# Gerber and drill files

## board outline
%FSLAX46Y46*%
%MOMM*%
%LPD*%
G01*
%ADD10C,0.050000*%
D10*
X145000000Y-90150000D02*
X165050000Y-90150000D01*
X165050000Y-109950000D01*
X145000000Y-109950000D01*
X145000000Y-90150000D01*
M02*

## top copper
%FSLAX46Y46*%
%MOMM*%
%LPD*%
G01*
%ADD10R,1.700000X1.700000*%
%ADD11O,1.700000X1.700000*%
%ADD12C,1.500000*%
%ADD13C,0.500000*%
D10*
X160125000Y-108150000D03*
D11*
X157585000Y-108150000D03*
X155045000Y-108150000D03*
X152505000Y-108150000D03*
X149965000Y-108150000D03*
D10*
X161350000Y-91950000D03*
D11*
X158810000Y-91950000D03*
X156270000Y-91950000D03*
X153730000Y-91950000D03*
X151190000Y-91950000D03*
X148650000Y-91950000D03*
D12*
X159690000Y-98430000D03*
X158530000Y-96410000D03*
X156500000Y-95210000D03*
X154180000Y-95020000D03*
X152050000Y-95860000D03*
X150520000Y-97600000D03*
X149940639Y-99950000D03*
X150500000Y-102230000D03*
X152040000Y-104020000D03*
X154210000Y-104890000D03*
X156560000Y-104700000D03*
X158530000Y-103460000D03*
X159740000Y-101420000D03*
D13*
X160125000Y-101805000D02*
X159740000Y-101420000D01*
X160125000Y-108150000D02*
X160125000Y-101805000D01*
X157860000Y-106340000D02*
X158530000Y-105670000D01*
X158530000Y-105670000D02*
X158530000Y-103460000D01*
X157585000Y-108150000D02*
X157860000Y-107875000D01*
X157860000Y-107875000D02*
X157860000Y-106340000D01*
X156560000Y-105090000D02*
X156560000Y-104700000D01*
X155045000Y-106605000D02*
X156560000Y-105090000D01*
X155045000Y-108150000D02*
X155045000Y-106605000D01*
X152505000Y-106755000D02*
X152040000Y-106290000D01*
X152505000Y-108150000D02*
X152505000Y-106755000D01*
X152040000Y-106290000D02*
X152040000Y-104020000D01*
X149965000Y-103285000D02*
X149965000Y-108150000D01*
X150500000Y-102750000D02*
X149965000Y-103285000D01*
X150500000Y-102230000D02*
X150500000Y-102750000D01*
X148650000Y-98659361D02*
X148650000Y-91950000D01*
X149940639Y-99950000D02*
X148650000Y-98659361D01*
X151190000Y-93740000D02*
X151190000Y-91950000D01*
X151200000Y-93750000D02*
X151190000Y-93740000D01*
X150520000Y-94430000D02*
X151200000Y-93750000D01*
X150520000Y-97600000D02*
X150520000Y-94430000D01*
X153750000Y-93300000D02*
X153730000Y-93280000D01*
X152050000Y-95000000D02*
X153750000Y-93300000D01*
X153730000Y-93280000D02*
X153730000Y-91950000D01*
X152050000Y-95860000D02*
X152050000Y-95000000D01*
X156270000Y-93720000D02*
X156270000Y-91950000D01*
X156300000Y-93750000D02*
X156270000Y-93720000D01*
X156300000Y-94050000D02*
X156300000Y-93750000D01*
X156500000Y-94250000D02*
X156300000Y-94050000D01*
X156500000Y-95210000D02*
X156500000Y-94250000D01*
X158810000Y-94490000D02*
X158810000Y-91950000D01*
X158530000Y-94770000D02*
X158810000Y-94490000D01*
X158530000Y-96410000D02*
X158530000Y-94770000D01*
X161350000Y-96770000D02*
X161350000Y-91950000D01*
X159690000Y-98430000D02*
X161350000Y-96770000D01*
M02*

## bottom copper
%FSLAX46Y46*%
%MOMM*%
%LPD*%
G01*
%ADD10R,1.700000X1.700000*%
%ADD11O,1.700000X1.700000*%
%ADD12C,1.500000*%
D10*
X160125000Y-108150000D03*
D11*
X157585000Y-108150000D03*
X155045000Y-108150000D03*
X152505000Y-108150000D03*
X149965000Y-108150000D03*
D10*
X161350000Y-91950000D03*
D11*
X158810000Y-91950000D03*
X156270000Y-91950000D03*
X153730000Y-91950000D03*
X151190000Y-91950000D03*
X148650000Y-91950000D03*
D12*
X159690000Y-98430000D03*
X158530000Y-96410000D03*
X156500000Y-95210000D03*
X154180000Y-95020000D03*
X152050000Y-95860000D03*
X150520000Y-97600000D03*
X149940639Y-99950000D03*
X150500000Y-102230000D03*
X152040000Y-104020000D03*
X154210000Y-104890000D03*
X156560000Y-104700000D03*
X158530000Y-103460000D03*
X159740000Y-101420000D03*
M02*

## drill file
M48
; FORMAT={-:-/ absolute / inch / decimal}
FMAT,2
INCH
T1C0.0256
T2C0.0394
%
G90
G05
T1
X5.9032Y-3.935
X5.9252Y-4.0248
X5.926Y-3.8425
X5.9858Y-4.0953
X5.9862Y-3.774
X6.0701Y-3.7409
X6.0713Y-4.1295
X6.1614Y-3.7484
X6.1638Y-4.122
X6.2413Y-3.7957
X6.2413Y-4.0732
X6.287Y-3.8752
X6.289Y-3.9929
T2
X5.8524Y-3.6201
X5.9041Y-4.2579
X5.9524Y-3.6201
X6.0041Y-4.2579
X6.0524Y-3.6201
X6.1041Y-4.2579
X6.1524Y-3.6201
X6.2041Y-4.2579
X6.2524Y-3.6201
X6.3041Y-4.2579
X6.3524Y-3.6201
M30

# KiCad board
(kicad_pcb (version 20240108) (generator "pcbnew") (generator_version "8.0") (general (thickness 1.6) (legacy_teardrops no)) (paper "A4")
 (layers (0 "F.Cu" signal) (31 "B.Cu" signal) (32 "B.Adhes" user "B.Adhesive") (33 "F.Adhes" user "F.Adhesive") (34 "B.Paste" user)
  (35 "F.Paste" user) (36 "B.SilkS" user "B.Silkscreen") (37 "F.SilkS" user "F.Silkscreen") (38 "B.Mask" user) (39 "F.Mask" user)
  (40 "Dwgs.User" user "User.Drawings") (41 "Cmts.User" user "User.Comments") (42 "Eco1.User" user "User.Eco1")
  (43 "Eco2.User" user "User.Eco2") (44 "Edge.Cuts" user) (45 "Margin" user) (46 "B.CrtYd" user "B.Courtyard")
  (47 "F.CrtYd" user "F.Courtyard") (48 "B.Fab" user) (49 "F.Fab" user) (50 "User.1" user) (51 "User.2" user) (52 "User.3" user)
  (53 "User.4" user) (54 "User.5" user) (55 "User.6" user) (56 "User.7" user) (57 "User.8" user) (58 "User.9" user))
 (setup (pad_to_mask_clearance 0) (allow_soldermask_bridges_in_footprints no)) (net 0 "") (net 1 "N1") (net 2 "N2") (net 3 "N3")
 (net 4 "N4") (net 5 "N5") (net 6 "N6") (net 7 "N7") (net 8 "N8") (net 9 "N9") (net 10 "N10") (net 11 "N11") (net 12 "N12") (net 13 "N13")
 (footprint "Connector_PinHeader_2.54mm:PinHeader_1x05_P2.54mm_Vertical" (layer "F.Cu") (at 160.125 108.15 -90)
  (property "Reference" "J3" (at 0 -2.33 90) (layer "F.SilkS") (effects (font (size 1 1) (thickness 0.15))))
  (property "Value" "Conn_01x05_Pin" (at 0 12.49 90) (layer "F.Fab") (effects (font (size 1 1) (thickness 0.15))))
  (pad "1" thru_hole rect (at 0 0 270) (size 1.7 1.7) (drill 1) (layers "*.Cu" "*.Mask") (remove_unused_layers no) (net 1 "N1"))
  (pad "2" thru_hole oval (at 0 2.54 270) (size 1.7 1.7) (drill 1) (layers "*.Cu" "*.Mask") (remove_unused_layers no) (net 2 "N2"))
  (pad "3" thru_hole oval (at 0 5.08 270) (size 1.7 1.7) (drill 1) (layers "*.Cu" "*.Mask") (remove_unused_layers no) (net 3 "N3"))
  (pad "4" thru_hole oval (at 0 7.62 270) (size 1.7 1.7) (drill 1) (layers "*.Cu" "*.Mask") (remove_unused_layers no) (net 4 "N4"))
  (pad "5" thru_hole oval (at 0 10.16 270) (size 1.7 1.7) (drill 1) (layers "*.Cu" "*.Mask") (remove_unused_layers no) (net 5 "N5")))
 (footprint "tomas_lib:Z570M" (layer "F.Cu") (at 154.95 99.95)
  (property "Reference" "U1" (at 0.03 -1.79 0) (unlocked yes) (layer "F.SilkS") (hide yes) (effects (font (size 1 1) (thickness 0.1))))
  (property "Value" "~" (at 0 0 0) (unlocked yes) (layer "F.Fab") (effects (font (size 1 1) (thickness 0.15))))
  (pad "1" thru_hole circle (at 4.74 -1.52) (size 1.5 1.5) (drill 0.65) (layers "*.Cu" "*.Mask") (remove_unused_layers no) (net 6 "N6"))
  (pad "2" thru_hole circle (at 3.58 -3.54) (size 1.5 1.5) (drill 0.65) (layers "*.Cu" "*.Mask") (remove_unused_layers no) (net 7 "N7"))
  (pad "3" thru_hole circle (at 1.55 -4.74) (size 1.5 1.5) (drill 0.65) (layers "*.Cu" "*.Mask") (remove_unused_layers no) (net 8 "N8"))
  (pad "4" thru_hole circle (at -0.77 -4.93) (size 1.5 1.5) (drill 0.65) (layers "*.Cu" "*.Mask") (remove_unused_layers no) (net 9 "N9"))
  (pad "5" thru_hole circle (at -2.9 -4.09) (size 1.5 1.5) (drill 0.65) (layers "*.Cu" "*.Mask") (remove_unused_layers no) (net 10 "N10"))
  (pad "6" thru_hole circle (at -4.43 -2.35) (size 1.5 1.5) (drill 0.65) (layers "*.Cu" "*.Mask") (remove_unused_layers no) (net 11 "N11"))
  (pad "7" thru_hole circle (at -5.009361 0) (size 1.5 1.5) (drill 0.65) (layers "*.Cu" "*.Mask") (remove_unused_layers no) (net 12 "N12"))
  (pad "8" thru_hole circle (at -4.45 2.28) (size 1.5 1.5) (drill 0.65) (layers "*.Cu" "*.Mask") (remove_unused_layers no) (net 5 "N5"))
  (pad "9" thru_hole circle (at -2.91 4.07) (size 1.5 1.5) (drill 0.65) (layers "*.Cu" "*.Mask") (remove_unused_layers no) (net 4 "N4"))
  (pad "10" thru_hole circle (at -0.74 4.94) (size 1.5 1.5) (drill 0.65) (layers "*.Cu" "*.Mask") (remove_unused_layers no) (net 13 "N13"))
  (pad "11" thru_hole circle (at 1.61 4.75) (size 1.5 1.5) (drill 0.65) (layers "*.Cu" "*.Mask") (remove_unused_layers no) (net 3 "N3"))
  (pad "12" thru_hole circle (at 3.58 3.51) (size 1.5 1.5) (drill 0.65) (layers "*.Cu" "*.Mask") (remove_unused_layers no) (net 2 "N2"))
  (pad "13" thru_hole circle (at 4.79 1.47) (size 1.5 1.5) (drill 0.65) (layers "*.Cu" "*.Mask") (remove_unused_layers no) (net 1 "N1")))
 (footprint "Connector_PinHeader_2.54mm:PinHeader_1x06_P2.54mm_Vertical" (layer "F.Cu") (at 161.35 91.95 -90)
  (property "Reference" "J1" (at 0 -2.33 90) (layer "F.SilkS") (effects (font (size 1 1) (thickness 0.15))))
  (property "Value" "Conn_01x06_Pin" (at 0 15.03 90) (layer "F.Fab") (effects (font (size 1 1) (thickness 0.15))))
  (pad "1" thru_hole rect (at 0 0 270) (size 1.7 1.7) (drill 1) (layers "*.Cu" "*.Mask") (remove_unused_layers no) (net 6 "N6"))
  (pad "2" thru_hole oval (at 0 2.54 270) (size 1.7 1.7) (drill 1) (layers "*.Cu" "*.Mask") (remove_unused_layers no) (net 7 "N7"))
  (pad "3" thru_hole oval (at 0 5.08 270) (size 1.7 1.7) (drill 1) (layers "*.Cu" "*.Mask") (remove_unused_layers no) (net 8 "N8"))
  (pad "4" thru_hole oval (at 0 7.62 270) (size 1.7 1.7) (drill 1) (layers "*.Cu" "*.Mask") (remove_unused_layers no) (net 10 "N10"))
  (pad "5" thru_hole oval (at 0 10.16 270) (size 1.7 1.7) (drill 1) (layers "*.Cu" "*.Mask") (remove_unused_layers no) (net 11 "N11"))
  (pad "6" thru_hole oval (at 0 12.7 270) (size 1.7 1.7) (drill 1) (layers "*.Cu" "*.Mask") (remove_unused_layers no) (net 12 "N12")))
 (gr_rect (start 145 90.15) (end 165.05 109.95) (stroke (width 0.05) (type default)) (fill none) (layer "Edge.Cuts"))
 (segment (start 149.965 103.285) (end 149.965 108.15) (width 0.5) (layer "F.Cu") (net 5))
 (segment (start 150.5 102.75) (end 149.965 103.285) (width 0.5) (layer "F.Cu") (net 5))
 (segment (start 150.5 102.23) (end 150.5 102.75) (width 0.5) (layer "F.Cu") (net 5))
 (segment (start 156.5 94.25) (end 156.3 94.05) (width 0.5) (layer "F.Cu") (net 8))
 (segment (start 156.3 93.75) (end 156.27 93.72) (width 0.5) (layer "F.Cu") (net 8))
 (segment (start 156.3 94.05) (end 156.3 93.75) (width 0.5) (layer "F.Cu") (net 8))
 (segment (start 156.27 93.72) (end 156.27 91.95) (width 0.5) (layer "F.Cu") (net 8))
 (segment (start 156.5 95.21) (end 156.5 94.25) (width 0.5) (layer "F.Cu") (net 8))
 (segment (start 160.125 108.15) (end 160.125 101.805) (width 0.5) (layer "F.Cu") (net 1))
 (segment (start 160.125 101.805) (end 159.74 101.42) (width 0.5) (layer "F.Cu") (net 1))
 (segment (start 158.81 94.49) (end 158.81 91.95) (width 0.5) (layer "F.Cu") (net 7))
 (segment (start 158.53 96.41) (end 158.53 94.77) (width 0.5) (layer "F.Cu") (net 7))
 (segment (start 158.53 94.77) (end 158.81 94.49) (width 0.5) (layer "F.Cu") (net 7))
 (segment (start 153.75 93.3) (end 153.73 93.28) (width 0.5) (layer "F.Cu") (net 10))
 (segment (start 153.73 93.28) (end 153.73 91.95) (width 0.5) (layer "F.Cu") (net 10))
 (segment (start 152.05 95.86) (end 152.05 95) (width 0.5) (layer "F.Cu") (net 10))
 (segment (start 152.05 95) (end 153.75 93.3) (width 0.5) (layer "F.Cu") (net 10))
 (segment (start 161.35 96.77) (end 161.35 91.95) (width 0.5) (layer "F.Cu") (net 6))
 (segment (start 159.69 98.43) (end 161.35 96.77) (width 0.5) (layer "F.Cu") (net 6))
 (segment (start 155.045 108.15) (end 155.045 106.605) (width 0.5) (layer "F.Cu") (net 3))
 (segment (start 155.045 106.605) (end 156.56 105.09) (width 0.5) (layer "F.Cu") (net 3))
 (segment (start 156.56 105.09) (end 156.56 104.7) (width 0.5) (layer "F.Cu") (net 3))
 (segment (start 150.52 94.43) (end 151.2 93.75) (width 0.5) (layer "F.Cu") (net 11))
 (segment (start 151.2 93.75) (end 151.19 93.74) (width 0.5) (layer "F.Cu") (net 11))
 (segment (start 151.19 93.74) (end 151.19 91.95) (width 0.5) (layer "F.Cu") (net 11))
 (segment (start 150.52 97.6) (end 150.52 94.43) (width 0.5) (layer "F.Cu") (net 11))
 (segment (start 157.86 107.875) (end 157.86 106.34) (width 0.5) (layer "F.Cu") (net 2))
 (segment (start 158.53 105.67) (end 158.53 103.46) (width 0.5) (layer "F.Cu") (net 2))
 (segment (start 157.585 108.15) (end 157.86 107.875) (width 0.5) (layer "F.Cu") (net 2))
 (segment (start 157.86 106.34) (end 158.53 105.67) (width 0.5) (layer "F.Cu") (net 2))
 (segment (start 152.505 106.755) (end 152.04 106.29) (width 0.5) (layer "F.Cu") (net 4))
 (segment (start 152.505 108.15) (end 152.505 106.755) (width 0.5) (layer "F.Cu") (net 4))
 (segment (start 152.04 106.29) (end 152.04 104.02) (width 0.5) (layer "F.Cu") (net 4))
 (segment (start 149.940639 99.95) (end 148.65 98.659361) (width 0.5) (layer "F.Cu") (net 12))
 (segment (start 148.65 98.659361) (end 148.65 91.95) (width 0.5) (layer "F.Cu") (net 12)))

